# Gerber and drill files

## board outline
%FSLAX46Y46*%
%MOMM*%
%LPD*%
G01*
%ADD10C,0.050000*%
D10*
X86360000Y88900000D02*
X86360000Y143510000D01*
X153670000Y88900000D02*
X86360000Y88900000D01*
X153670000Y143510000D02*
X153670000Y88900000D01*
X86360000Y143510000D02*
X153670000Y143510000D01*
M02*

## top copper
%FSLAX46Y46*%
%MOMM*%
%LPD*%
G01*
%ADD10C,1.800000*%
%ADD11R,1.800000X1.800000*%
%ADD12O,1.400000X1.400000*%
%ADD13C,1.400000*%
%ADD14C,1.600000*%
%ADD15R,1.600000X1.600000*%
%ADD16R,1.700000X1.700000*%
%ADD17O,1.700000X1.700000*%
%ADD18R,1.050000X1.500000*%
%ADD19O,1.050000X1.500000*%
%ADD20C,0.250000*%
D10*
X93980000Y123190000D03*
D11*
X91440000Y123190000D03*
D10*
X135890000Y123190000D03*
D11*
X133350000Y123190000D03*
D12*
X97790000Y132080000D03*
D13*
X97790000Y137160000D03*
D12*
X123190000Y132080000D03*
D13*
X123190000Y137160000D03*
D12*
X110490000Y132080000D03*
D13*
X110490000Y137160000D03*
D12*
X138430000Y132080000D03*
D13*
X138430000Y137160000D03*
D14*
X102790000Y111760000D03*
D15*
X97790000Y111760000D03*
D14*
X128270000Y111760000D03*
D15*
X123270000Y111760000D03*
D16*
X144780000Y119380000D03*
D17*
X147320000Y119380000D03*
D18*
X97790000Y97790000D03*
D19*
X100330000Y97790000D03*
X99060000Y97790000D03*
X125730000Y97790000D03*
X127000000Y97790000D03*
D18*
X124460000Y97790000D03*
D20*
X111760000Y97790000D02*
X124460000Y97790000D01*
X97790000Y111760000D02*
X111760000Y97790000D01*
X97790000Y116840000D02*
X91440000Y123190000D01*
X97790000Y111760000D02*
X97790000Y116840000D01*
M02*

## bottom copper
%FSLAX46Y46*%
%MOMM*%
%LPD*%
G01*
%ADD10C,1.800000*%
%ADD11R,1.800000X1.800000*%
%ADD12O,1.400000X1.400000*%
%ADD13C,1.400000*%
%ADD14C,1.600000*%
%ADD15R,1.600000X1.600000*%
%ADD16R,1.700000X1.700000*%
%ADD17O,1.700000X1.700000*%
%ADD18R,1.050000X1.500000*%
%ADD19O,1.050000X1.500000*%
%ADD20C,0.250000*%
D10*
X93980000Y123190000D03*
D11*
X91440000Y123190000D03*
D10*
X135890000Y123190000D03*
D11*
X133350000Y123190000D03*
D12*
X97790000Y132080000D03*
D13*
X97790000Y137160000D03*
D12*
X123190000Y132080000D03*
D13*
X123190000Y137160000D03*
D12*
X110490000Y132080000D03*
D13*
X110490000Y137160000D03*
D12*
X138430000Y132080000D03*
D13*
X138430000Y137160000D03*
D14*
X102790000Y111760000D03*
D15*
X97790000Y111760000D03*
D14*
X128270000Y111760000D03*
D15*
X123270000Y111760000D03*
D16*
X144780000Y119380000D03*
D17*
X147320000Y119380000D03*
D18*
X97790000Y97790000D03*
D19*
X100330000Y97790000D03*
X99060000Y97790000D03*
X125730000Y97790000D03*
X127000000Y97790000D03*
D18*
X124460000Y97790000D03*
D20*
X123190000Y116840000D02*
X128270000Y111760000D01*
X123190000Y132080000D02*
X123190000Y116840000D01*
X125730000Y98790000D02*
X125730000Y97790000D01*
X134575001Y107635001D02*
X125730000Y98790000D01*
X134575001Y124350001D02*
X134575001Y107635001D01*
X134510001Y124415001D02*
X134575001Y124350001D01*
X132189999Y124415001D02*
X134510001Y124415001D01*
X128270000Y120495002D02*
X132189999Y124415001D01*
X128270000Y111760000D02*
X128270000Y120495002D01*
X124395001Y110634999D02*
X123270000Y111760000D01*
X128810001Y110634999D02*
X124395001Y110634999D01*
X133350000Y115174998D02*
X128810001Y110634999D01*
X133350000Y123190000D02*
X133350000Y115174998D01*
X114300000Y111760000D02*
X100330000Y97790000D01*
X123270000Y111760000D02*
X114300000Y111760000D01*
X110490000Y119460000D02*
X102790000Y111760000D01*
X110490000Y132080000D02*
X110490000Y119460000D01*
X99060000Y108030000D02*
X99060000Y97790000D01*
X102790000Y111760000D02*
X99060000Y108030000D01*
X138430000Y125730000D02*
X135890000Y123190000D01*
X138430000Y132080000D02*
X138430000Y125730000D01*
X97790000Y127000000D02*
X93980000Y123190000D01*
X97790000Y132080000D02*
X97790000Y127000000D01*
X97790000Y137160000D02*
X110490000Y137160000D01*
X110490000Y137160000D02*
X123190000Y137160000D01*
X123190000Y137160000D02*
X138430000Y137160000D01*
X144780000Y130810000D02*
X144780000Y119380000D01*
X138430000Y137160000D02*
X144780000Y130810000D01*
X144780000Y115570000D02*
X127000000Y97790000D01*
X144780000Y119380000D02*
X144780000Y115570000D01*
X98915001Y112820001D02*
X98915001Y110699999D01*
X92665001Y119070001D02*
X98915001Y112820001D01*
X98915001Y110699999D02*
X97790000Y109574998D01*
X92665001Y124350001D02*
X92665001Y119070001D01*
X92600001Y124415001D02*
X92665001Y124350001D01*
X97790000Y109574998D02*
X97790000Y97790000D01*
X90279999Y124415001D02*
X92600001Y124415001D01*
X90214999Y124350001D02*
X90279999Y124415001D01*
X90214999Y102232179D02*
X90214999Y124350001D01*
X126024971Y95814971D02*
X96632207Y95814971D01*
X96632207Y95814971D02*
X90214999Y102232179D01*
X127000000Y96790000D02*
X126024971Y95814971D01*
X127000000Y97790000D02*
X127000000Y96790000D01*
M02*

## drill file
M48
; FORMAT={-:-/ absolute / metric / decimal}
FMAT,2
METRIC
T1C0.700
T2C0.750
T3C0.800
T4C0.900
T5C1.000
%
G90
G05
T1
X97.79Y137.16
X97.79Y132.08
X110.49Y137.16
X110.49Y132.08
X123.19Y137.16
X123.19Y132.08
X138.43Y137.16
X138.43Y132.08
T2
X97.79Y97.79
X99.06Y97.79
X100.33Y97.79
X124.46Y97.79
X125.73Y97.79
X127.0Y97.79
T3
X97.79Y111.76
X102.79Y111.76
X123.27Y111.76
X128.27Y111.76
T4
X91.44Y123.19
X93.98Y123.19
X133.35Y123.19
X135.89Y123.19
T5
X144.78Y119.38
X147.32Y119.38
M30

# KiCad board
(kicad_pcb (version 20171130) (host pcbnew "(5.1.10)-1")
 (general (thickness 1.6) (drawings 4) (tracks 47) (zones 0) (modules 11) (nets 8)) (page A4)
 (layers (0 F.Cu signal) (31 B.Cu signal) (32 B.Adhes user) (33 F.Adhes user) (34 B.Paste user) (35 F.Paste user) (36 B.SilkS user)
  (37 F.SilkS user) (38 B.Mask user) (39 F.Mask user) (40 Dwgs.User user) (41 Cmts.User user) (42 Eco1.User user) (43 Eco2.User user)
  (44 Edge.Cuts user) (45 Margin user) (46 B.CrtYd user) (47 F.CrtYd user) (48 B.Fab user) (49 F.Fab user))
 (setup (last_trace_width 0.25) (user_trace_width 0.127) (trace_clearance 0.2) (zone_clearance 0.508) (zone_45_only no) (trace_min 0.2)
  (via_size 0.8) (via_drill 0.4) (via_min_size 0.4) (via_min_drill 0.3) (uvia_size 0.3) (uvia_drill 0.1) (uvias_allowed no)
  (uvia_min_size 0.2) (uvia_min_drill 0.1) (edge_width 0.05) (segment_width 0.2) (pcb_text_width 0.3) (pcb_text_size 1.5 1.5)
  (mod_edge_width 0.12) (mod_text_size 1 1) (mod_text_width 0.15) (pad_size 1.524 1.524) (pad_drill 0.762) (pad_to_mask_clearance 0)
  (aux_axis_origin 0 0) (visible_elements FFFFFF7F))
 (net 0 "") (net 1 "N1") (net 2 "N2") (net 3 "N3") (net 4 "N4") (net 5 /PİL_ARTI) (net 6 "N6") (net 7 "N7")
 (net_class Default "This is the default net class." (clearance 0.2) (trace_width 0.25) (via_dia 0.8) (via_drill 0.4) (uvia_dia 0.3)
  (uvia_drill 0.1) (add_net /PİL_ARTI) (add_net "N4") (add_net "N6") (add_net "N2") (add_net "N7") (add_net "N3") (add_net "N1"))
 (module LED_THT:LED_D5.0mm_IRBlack (layer F.Cu) (at 91.44 -123.19)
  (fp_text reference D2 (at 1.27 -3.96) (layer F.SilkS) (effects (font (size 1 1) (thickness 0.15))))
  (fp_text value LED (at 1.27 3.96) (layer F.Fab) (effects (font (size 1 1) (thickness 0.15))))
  (pad 2 thru_hole circle (at 2.54 0) (size 1.8 1.8) (drill 0.9) (layers *.Cu *.Mask) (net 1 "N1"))
  (pad 1 thru_hole rect (at 0 0) (size 1.8 1.8) (drill 0.9) (layers *.Cu *.Mask) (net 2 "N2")))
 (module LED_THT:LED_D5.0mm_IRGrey (layer F.Cu) (at 133.35 -123.19)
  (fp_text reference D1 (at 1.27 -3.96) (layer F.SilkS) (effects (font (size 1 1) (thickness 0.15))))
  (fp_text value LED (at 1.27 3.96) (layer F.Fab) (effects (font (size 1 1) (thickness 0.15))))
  (pad 2 thru_hole circle (at 2.54 0) (size 1.8 1.8) (drill 0.9) (layers *.Cu *.Mask) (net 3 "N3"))
  (pad 1 thru_hole rect (at 0 0) (size 1.8 1.8) (drill 0.9) (layers *.Cu *.Mask) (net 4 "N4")))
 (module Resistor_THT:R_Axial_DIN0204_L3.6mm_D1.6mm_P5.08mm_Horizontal (layer F.Cu) (at 97.79 -137.16 270)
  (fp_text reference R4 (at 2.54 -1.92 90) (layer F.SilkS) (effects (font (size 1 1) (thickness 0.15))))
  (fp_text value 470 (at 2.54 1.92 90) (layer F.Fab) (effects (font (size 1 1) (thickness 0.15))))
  (pad 2 thru_hole oval (at 5.08 0 270) (size 1.4 1.4) (drill 0.7) (layers *.Cu *.Mask) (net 1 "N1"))
  (pad 1 thru_hole circle (at 0 0 270) (size 1.4 1.4) (drill 0.7) (layers *.Cu *.Mask) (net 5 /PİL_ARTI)))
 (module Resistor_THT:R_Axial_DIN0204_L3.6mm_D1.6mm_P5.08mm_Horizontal (layer F.Cu) (at 123.19 -137.16 270)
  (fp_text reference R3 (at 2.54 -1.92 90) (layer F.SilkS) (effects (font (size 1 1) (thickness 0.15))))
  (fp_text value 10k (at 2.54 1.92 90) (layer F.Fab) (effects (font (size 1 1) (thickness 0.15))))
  (pad 2 thru_hole oval (at 5.08 0 270) (size 1.4 1.4) (drill 0.7) (layers *.Cu *.Mask) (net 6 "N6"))
  (pad 1 thru_hole circle (at 0 0 270) (size 1.4 1.4) (drill 0.7) (layers *.Cu *.Mask) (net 5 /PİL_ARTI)))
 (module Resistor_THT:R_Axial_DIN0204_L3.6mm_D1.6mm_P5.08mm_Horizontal (layer F.Cu) (at 110.49 -137.16 270)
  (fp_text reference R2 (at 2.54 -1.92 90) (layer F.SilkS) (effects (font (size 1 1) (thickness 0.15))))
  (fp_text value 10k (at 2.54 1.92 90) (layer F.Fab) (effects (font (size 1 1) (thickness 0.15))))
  (pad 2 thru_hole oval (at 5.08 0 270) (size 1.4 1.4) (drill 0.7) (layers *.Cu *.Mask) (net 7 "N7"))
  (pad 1 thru_hole circle (at 0 0 270) (size 1.4 1.4) (drill 0.7) (layers *.Cu *.Mask) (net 5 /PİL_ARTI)))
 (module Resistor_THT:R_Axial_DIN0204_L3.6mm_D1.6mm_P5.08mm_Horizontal (layer F.Cu) (at 138.43 -137.16 270)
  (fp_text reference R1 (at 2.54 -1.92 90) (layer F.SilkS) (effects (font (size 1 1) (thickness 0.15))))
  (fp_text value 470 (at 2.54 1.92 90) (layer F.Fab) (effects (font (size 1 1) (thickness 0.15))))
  (pad 2 thru_hole oval (at 5.08 0 270) (size 1.4 1.4) (drill 0.7) (layers *.Cu *.Mask) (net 3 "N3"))
  (pad 1 thru_hole circle (at 0 0 270) (size 1.4 1.4) (drill 0.7) (layers *.Cu *.Mask) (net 5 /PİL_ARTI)))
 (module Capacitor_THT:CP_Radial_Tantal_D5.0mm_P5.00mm (layer F.Cu) (at 97.79 -111.76)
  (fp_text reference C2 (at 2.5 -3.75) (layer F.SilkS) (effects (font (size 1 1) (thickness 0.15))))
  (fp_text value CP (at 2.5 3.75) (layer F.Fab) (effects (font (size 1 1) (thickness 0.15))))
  (pad 2 thru_hole circle (at 5 0) (size 1.6 1.6) (drill 0.8) (layers *.Cu *.Mask) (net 7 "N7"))
  (pad 1 thru_hole rect (at 0 0) (size 1.6 1.6) (drill 0.8) (layers *.Cu *.Mask) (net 2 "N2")))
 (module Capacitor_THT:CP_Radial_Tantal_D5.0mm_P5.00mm (layer F.Cu) (at 123.27 -111.76)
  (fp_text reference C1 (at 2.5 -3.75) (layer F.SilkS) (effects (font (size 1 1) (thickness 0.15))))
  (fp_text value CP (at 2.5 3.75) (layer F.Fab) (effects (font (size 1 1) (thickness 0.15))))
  (pad 2 thru_hole circle (at 5 0) (size 1.6 1.6) (drill 0.8) (layers *.Cu *.Mask) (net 6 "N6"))
  (pad 1 thru_hole rect (at 0 0) (size 1.6 1.6) (drill 0.8) (layers *.Cu *.Mask) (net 4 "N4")))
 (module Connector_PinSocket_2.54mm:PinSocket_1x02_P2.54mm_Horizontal (layer F.Cu) (at 144.78 -119.38 90)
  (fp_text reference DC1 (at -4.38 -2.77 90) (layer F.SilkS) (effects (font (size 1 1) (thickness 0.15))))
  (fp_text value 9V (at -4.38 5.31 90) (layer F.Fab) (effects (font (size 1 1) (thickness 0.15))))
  (pad 1 thru_hole rect (at 0 0 90) (size 1.7 1.7) (drill 1) (layers *.Cu *.Mask) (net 5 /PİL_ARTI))
  (pad 2 thru_hole oval (at 0 2.54 90) (size 1.7 1.7) (drill 1) (layers *.Cu *.Mask) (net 5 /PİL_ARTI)))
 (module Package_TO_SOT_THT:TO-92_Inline (layer F.Cu) (at 97.79 -97.79)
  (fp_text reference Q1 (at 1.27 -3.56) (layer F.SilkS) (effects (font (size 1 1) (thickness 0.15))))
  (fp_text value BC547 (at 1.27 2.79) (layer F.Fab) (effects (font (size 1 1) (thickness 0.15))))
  (pad 1 thru_hole rect (at 0 0) (size 1.05 1.5) (drill 0.75) (layers *.Cu *.Mask) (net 5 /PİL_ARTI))
  (pad 3 thru_hole oval (at 2.54 0) (size 1.05 1.5) (drill 0.75) (layers *.Cu *.Mask) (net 4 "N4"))
  (pad 2 thru_hole oval (at 1.27 0) (size 1.05 1.5) (drill 0.75) (layers *.Cu *.Mask) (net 7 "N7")))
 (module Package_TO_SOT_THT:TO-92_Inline (layer F.Cu) (at 124.46 -97.79)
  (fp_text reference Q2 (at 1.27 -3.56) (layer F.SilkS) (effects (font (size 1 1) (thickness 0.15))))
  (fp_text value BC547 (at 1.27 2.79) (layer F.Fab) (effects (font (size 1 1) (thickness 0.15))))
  (pad 2 thru_hole oval (at 1.27 0) (size 1.05 1.5) (drill 0.75) (layers *.Cu *.Mask) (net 6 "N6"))
  (pad 3 thru_hole oval (at 2.54 0) (size 1.05 1.5) (drill 0.75) (layers *.Cu *.Mask) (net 5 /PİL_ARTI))
  (pad 1 thru_hole rect (at 0 0) (size 1.05 1.5) (drill 0.75) (layers *.Cu *.Mask) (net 2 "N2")))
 (gr_line (start 86.36 -88.9) (end 86.36 -143.51) (layer Edge.Cuts) (width 0.05))
 (gr_line (start 153.67 -88.9) (end 86.36 -88.9) (layer Edge.Cuts) (width 0.05))
 (gr_line (start 153.67 -143.51) (end 153.67 -88.9) (layer Edge.Cuts) (width 0.05))
 (gr_line (start 86.36 -143.51) (end 153.67 -143.51) (layer Edge.Cuts) (width 0.05))
 (segment (start 123.19 -116.84) (end 128.27 -111.76) (width 0.25) (layer B.Cu) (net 6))
 (segment (start 123.19 -132.08) (end 123.19 -116.84) (width 0.25) (layer B.Cu) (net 6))
 (segment (start 125.73 -98.79) (end 125.73 -97.79) (width 0.25) (layer B.Cu) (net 6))
 (segment (start 134.575001 -107.635001) (end 125.73 -98.79) (width 0.25) (layer B.Cu) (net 6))
 (segment (start 134.575001 -124.350001) (end 134.575001 -107.635001) (width 0.25) (layer B.Cu) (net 6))
 (segment (start 134.510001 -124.415001) (end 134.575001 -124.350001) (width 0.25) (layer B.Cu) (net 6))
 (segment (start 132.189999 -124.415001) (end 134.510001 -124.415001) (width 0.25) (layer B.Cu) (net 6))
 (segment (start 128.27 -120.495002) (end 132.189999 -124.415001) (width 0.25) (layer B.Cu) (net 6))
 (segment (start 128.27 -111.76) (end 128.27 -120.495002) (width 0.25) (layer B.Cu) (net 6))
 (segment (start 124.395001 -110.634999) (end 123.27 -111.76) (width 0.25) (layer B.Cu) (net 4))
 (segment (start 128.810001 -110.634999) (end 124.395001 -110.634999) (width 0.25) (layer B.Cu) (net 4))
 (segment (start 133.35 -115.174998) (end 128.810001 -110.634999) (width 0.25) (layer B.Cu) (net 4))
 (segment (start 133.35 -123.19) (end 133.35 -115.174998) (width 0.25) (layer B.Cu) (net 4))
 (segment (start 114.3 -111.76) (end 100.33 -97.79) (width 0.25) (layer B.Cu) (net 4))
 (segment (start 123.27 -111.76) (end 114.3 -111.76) (width 0.25) (layer B.Cu) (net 4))
 (segment (start 111.76 -97.79) (end 124.46 -97.79) (width 0.25) (layer F.Cu) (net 2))
 (segment (start 97.79 -111.76) (end 111.76 -97.79) (width 0.25) (layer F.Cu) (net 2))
 (segment (start 97.79 -116.84) (end 91.44 -123.19) (width 0.25) (layer F.Cu) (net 2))
 (segment (start 97.79 -111.76) (end 97.79 -116.84) (width 0.25) (layer F.Cu) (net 2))
 (segment (start 110.49 -119.46) (end 102.79 -111.76) (width 0.25) (layer B.Cu) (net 7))
 (segment (start 110.49 -132.08) (end 110.49 -119.46) (width 0.25) (layer B.Cu) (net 7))
 (segment (start 99.06 -108.03) (end 99.06 -97.79) (width 0.25) (layer B.Cu) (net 7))
 (segment (start 102.79 -111.76) (end 99.06 -108.03) (width 0.25) (layer B.Cu) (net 7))
 (segment (start 138.43 -125.73) (end 135.89 -123.19) (width 0.25) (layer B.Cu) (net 3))
 (segment (start 138.43 -132.08) (end 138.43 -125.73) (width 0.25) (layer B.Cu) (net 3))
 (segment (start 97.79 -127) (end 93.98 -123.19) (width 0.25) (layer B.Cu) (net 1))
 (segment (start 97.79 -132.08) (end 97.79 -127) (width 0.25) (layer B.Cu) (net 1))
 (segment (start 97.79 -137.16) (end 110.49 -137.16) (width 0.25) (layer B.Cu) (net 5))
 (segment (start 110.49 -137.16) (end 123.19 -137.16) (width 0.25) (layer B.Cu) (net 5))
 (segment (start 123.19 -137.16) (end 138.43 -137.16) (width 0.25) (layer B.Cu) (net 5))
 (segment (start 144.78 -130.81) (end 144.78 -119.38) (width 0.25) (layer B.Cu) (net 5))
 (segment (start 138.43 -137.16) (end 144.78 -130.81) (width 0.25) (layer B.Cu) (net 5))
 (segment (start 144.78 -115.57) (end 127 -97.79) (width 0.25) (layer B.Cu) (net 5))
 (segment (start 144.78 -119.38) (end 144.78 -115.57) (width 0.25) (layer B.Cu) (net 5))
 (segment (start 98.915001 -112.820001) (end 98.915001 -110.699999) (width 0.25) (layer B.Cu) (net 5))
 (segment (start 92.665001 -119.070001) (end 98.915001 -112.820001) (width 0.25) (layer B.Cu) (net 5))
 (segment (start 98.915001 -110.699999) (end 97.79 -109.574998) (width 0.25) (layer B.Cu) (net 5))
 (segment (start 92.665001 -124.350001) (end 92.665001 -119.070001) (width 0.25) (layer B.Cu) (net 5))
 (segment (start 92.600001 -124.415001) (end 92.665001 -124.350001) (width 0.25) (layer B.Cu) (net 5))
 (segment (start 97.79 -109.574998) (end 97.79 -97.79) (width 0.25) (layer B.Cu) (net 5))
 (segment (start 90.279999 -124.415001) (end 92.600001 -124.415001) (width 0.25) (layer B.Cu) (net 5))
 (segment (start 90.214999 -124.350001) (end 90.279999 -124.415001) (width 0.25) (layer B.Cu) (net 5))
 (segment (start 90.214999 -102.232179) (end 90.214999 -124.350001) (width 0.25) (layer B.Cu) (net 5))
 (segment (start 126.024971 -95.814971) (end 96.632207 -95.814971) (width 0.25) (layer B.Cu) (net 5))
 (segment (start 96.632207 -95.814971) (end 90.214999 -102.232179) (width 0.25) (layer B.Cu) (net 5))
 (segment (start 127 -96.79) (end 126.024971 -95.814971) (width 0.25) (layer B.Cu) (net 5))
 (segment (start 127 -97.79) (end 127 -96.79) (width 0.25) (layer B.Cu) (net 5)))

